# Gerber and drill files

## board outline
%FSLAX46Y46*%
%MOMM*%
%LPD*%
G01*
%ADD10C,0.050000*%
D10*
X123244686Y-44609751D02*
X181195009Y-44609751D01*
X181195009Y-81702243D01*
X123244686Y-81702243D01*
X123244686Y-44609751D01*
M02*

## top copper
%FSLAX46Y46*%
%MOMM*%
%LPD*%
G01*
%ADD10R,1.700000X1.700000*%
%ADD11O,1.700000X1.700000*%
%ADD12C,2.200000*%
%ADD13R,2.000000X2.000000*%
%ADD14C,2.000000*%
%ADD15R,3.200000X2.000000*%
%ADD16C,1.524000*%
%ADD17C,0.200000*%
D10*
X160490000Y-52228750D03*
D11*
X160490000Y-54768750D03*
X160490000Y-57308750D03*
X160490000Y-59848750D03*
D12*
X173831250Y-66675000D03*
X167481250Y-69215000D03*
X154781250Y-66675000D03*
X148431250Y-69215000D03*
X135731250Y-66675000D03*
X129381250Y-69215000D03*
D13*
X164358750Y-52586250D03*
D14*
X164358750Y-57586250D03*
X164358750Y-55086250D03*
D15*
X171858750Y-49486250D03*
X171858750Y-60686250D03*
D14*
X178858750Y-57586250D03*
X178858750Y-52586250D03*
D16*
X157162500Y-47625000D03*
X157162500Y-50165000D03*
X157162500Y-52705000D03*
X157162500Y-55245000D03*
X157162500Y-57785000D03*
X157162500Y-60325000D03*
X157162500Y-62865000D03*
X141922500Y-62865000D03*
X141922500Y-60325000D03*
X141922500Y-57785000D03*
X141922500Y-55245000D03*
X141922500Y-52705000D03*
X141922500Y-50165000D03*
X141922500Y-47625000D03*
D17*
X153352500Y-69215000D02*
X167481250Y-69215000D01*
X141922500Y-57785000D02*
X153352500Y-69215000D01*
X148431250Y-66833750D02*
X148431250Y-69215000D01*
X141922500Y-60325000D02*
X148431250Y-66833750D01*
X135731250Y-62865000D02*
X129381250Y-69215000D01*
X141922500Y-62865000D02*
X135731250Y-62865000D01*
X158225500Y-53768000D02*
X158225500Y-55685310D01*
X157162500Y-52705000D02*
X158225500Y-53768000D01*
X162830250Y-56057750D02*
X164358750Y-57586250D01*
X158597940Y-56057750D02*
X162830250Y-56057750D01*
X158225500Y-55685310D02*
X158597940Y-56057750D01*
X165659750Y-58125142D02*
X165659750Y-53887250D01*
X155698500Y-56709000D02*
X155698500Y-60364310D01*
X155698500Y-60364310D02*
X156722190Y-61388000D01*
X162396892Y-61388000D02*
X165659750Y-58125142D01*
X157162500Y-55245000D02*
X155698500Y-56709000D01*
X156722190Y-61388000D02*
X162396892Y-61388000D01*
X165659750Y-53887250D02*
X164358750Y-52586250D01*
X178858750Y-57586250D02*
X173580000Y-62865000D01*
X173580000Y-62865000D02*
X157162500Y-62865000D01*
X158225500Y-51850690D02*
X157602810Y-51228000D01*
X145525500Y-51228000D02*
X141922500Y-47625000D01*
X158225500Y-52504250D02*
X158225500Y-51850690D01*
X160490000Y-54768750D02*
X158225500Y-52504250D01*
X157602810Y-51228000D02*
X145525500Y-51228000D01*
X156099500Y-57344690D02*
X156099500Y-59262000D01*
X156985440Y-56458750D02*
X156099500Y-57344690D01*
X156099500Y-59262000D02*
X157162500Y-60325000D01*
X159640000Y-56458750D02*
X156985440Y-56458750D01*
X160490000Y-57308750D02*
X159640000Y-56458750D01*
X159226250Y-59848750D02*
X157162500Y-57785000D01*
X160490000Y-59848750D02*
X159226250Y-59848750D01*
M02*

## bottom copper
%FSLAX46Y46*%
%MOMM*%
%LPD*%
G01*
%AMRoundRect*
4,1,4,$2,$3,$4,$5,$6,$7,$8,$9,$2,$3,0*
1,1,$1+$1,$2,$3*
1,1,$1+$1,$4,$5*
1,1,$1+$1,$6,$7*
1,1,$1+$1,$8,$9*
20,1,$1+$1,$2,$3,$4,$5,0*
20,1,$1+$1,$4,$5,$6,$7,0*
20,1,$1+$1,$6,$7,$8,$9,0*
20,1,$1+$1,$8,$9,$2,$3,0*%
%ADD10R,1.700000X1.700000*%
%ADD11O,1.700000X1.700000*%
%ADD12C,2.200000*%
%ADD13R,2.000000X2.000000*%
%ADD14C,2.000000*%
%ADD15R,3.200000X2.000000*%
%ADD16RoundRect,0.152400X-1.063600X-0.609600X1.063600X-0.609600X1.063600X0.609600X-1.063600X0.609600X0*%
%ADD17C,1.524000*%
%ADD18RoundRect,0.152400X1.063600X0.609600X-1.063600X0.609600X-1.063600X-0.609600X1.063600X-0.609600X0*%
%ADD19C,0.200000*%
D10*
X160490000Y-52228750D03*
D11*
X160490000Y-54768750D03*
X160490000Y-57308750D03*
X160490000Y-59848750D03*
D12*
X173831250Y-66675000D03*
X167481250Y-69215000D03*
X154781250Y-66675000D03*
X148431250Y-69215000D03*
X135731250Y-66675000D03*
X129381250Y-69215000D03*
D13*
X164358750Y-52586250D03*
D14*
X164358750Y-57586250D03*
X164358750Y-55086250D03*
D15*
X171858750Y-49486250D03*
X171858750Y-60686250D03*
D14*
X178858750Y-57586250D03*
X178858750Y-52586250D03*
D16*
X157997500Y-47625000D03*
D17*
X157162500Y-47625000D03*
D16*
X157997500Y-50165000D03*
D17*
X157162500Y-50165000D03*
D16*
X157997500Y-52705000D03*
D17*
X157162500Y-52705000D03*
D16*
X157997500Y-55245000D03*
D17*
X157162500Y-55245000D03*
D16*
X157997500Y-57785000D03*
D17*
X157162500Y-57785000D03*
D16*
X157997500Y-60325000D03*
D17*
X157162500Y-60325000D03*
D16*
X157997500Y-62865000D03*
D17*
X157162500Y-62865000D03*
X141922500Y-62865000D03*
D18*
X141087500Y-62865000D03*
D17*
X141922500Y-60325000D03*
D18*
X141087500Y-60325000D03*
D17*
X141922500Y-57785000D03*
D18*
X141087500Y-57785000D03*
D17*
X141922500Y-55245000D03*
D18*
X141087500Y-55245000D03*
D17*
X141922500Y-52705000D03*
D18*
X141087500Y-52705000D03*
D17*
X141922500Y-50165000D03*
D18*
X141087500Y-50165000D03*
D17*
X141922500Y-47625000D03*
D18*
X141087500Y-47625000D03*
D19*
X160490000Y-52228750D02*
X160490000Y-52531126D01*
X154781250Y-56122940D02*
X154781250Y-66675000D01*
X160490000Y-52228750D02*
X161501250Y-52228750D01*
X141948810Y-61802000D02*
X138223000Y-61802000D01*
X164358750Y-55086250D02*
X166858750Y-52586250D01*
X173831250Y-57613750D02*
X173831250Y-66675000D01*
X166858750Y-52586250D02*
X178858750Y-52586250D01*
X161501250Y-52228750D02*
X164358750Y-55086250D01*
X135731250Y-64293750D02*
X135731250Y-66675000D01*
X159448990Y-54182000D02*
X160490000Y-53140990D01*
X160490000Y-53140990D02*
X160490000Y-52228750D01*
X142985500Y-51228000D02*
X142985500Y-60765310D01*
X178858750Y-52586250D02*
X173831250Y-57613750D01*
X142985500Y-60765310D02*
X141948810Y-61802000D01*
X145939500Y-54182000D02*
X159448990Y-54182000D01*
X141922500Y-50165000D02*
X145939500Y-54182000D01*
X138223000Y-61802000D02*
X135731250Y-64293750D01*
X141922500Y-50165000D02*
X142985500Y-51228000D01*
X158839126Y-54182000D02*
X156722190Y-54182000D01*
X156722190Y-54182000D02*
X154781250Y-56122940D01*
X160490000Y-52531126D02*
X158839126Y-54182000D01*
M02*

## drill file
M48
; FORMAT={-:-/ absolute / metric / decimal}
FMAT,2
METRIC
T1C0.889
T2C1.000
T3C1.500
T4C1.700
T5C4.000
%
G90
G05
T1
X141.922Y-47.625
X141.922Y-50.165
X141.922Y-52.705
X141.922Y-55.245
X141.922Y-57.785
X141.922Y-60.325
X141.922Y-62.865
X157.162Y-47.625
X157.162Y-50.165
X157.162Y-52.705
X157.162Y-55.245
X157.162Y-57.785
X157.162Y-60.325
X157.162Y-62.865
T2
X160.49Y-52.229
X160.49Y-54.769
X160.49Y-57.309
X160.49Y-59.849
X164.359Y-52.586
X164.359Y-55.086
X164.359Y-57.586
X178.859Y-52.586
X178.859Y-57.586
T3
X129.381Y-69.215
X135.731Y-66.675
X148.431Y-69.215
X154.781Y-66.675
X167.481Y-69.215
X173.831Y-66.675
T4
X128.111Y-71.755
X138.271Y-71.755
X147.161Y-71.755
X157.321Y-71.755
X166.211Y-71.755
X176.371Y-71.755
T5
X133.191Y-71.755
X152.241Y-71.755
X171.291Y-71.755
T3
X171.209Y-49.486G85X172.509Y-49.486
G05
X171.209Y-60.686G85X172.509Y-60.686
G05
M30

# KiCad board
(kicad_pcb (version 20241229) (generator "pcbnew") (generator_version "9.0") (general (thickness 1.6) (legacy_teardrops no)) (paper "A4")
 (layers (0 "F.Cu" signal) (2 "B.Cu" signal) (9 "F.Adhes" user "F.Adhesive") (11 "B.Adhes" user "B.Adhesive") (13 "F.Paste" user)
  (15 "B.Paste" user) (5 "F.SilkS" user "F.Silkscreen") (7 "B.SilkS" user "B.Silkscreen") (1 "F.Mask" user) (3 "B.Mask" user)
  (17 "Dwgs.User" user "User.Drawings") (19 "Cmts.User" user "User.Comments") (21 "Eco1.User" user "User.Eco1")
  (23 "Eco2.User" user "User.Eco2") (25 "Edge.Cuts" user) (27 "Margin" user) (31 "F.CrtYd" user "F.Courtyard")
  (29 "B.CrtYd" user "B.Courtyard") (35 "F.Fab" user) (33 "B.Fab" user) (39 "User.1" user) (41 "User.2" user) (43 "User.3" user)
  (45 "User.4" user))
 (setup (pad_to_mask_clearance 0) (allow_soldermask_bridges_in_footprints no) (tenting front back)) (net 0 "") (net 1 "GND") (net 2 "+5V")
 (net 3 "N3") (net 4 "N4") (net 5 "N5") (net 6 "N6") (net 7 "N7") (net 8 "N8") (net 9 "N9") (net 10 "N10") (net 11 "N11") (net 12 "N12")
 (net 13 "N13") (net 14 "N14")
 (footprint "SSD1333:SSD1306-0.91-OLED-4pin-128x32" (layer "F.Cu") (at 123.99 50.03875)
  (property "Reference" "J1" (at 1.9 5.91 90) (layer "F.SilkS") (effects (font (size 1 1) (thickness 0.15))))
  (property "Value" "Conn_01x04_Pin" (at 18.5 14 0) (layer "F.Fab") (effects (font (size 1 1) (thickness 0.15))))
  (pad "1" thru_hole rect (at 36.5 2.19) (size 1.7 1.7) (drill 1) (layers "*.Cu" "*.Mask") (remove_unused_layers no) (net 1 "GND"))
  (pad "2" thru_hole oval (at 36.5 4.73) (size 1.7 1.7) (drill 1) (layers "*.Cu" "*.Mask") (remove_unused_layers no) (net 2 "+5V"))
  (pad "3" thru_hole oval (at 36.5 7.27) (size 1.7 1.7) (drill 1) (layers "*.Cu" "*.Mask") (remove_unused_layers no) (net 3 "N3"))
  (pad "4" thru_hole oval (at 36.5 9.81) (size 1.7 1.7) (drill 1) (layers "*.Cu" "*.Mask") (remove_unused_layers no) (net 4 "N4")))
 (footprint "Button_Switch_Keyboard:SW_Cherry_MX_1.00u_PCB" (layer "F.Cu") (at 173.83125 66.675)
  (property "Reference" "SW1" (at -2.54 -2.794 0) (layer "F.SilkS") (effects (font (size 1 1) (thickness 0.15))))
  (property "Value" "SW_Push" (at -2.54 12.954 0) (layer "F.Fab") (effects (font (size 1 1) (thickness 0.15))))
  (pad "" np_thru_hole circle (at -7.62 5.08) (size 1.7 1.7) (drill 1.7) (layers "*.Cu" "*.Mask"))
  (pad "" np_thru_hole circle (at -2.54 5.08) (size 4 4) (drill 4) (layers "*.Cu" "*.Mask"))
  (pad "" np_thru_hole circle (at 2.54 5.08) (size 1.7 1.7) (drill 1.7) (layers "*.Cu" "*.Mask"))
  (pad "1" thru_hole circle (at 0 0) (size 2.2 2.2) (drill 1.5) (layers "*.Cu" "*.Mask") (remove_unused_layers no) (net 1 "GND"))
  (pad "2" thru_hole circle (at -6.35 2.54) (size 2.2 2.2) (drill 1.5) (layers "*.Cu" "*.Mask") (remove_unused_layers no) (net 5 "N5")))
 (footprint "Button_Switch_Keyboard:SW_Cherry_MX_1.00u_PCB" (layer "F.Cu") (at 154.78125 66.675)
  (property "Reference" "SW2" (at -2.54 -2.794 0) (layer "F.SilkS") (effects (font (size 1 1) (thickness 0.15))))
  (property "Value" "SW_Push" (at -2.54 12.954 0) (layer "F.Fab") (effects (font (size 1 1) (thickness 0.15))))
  (pad "" np_thru_hole circle (at -7.62 5.08) (size 1.7 1.7) (drill 1.7) (layers "*.Cu" "*.Mask"))
  (pad "" np_thru_hole circle (at -2.54 5.08) (size 4 4) (drill 4) (layers "*.Cu" "*.Mask"))
  (pad "" np_thru_hole circle (at 2.54 5.08) (size 1.7 1.7) (drill 1.7) (layers "*.Cu" "*.Mask"))
  (pad "1" thru_hole circle (at 0 0) (size 2.2 2.2) (drill 1.5) (layers "*.Cu" "*.Mask") (remove_unused_layers no) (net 1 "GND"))
  (pad "2" thru_hole circle (at -6.35 2.54) (size 2.2 2.2) (drill 1.5) (layers "*.Cu" "*.Mask") (remove_unused_layers no) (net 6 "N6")))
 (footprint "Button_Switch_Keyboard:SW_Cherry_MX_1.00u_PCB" (layer "F.Cu") (at 135.73125 66.675)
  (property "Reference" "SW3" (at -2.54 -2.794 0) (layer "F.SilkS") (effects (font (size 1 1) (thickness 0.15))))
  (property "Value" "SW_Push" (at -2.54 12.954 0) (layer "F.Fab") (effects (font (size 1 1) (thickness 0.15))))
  (pad "" np_thru_hole circle (at -7.62 5.08) (size 1.7 1.7) (drill 1.7) (layers "*.Cu" "*.Mask"))
  (pad "" np_thru_hole circle (at -2.54 5.08) (size 4 4) (drill 4) (layers "*.Cu" "*.Mask"))
  (pad "" np_thru_hole circle (at 2.54 5.08) (size 1.7 1.7) (drill 1.7) (layers "*.Cu" "*.Mask"))
  (pad "1" thru_hole circle (at 0 0) (size 2.2 2.2) (drill 1.5) (layers "*.Cu" "*.Mask") (remove_unused_layers no) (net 1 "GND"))
  (pad "2" thru_hole circle (at -6.35 2.54) (size 2.2 2.2) (drill 1.5) (layers "*.Cu" "*.Mask") (remove_unused_layers no) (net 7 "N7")))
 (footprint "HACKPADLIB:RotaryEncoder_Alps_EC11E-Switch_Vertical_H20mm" (layer "F.Cu") (at 164.35875 52.58625)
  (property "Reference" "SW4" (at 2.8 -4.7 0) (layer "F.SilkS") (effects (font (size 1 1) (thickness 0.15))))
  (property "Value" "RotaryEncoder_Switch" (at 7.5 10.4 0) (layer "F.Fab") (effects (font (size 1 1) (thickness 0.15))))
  (pad "A" thru_hole rect (at 0 0) (size 2 2) (drill 1) (layers "*.Cu" "*.Mask") (remove_unused_layers no) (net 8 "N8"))
  (pad "B" thru_hole circle (at 0 5) (size 2 2) (drill 1) (layers "*.Cu" "*.Mask") (remove_unused_layers no) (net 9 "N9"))
  (pad "C" thru_hole circle (at 0 2.5) (size 2 2) (drill 1) (layers "*.Cu" "*.Mask") (remove_unused_layers no) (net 1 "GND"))
  (pad "MP" thru_hole rect (at 7.5 -3.1) (size 3.2 2) (drill oval 2.8 1.5) (layers "*.Cu" "*.Mask") (remove_unused_layers no))
  (pad "MP" thru_hole rect (at 7.5 8.1) (size 3.2 2) (drill oval 2.8 1.5) (layers "*.Cu" "*.Mask") (remove_unused_layers no))
  (pad "S1" thru_hole circle (at 14.5 5) (size 2 2) (drill 1) (layers "*.Cu" "*.Mask") (remove_unused_layers no) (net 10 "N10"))
  (pad "S2" thru_hole circle (at 14.5 0) (size 2 2) (drill 1) (layers "*.Cu" "*.Mask") (remove_unused_layers no) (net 1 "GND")))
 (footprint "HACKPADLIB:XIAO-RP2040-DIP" (layer "B.Cu") (at 149.5425 55.245 180)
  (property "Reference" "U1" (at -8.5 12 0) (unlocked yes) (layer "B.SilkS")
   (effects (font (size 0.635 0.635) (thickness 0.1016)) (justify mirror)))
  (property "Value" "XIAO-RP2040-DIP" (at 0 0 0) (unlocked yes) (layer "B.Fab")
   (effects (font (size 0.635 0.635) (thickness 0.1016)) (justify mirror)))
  (pad "1" smd roundrect (at -8.455 7.62) (size 2.432 1.524) (layers "B.Cu" "B.Mask") (roundrect_rratio 0.1) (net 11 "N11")
   (thermal_bridge_angle 45))
  (pad "1" thru_hole circle (at -7.62 7.62) (size 1.524 1.524) (drill 0.889) (layers "*.Cu" "*.Mask") (remove_unused_layers no)
   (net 11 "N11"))
  (pad "2" smd roundrect (at -8.455 5.08) (size 2.432 1.524) (layers "B.Cu" "B.Mask") (roundrect_rratio 0.1) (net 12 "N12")
   (thermal_bridge_angle 45))
  (pad "2" thru_hole circle (at -7.62 5.08) (size 1.524 1.524) (drill 0.889) (layers "*.Cu" "*.Mask") (remove_unused_layers no)
   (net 12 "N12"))
  (pad "3" smd roundrect (at -8.455 2.54) (size 2.432 1.524) (layers "B.Cu" "B.Mask") (roundrect_rratio 0.1) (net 9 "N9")
   (thermal_bridge_angle 45))
  (pad "3" thru_hole circle (at -7.62 2.54) (size 1.524 1.524) (drill 0.889) (layers "*.Cu" "*.Mask") (remove_unused_layers no) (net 9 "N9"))
  (pad "4" smd roundrect (at -8.455 0) (size 2.432 1.524) (layers "B.Cu" "B.Mask") (roundrect_rratio 0.1) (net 8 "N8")
   (thermal_bridge_angle 45))
  (pad "4" thru_hole circle (at -7.62 0) (size 1.524 1.524) (drill 0.889) (layers "*.Cu" "*.Mask") (remove_unused_layers no) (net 8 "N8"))
  (pad "5" smd roundrect (at -8.455 -2.54) (size 2.432 1.524) (layers "B.Cu" "B.Mask") (roundrect_rratio 0.1) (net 4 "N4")
   (thermal_bridge_angle 45))
  (pad "5" thru_hole circle (at -7.62 -2.54) (size 1.524 1.524) (drill 0.889) (layers "*.Cu" "*.Mask") (remove_unused_layers no)
   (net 4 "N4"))
  (pad "6" smd roundrect (at -8.455 -5.08) (size 2.432 1.524) (layers "B.Cu" "B.Mask") (roundrect_rratio 0.1) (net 3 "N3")
   (thermal_bridge_angle 45))
  (pad "6" thru_hole circle (at -7.62 -5.08) (size 1.524 1.524) (drill 0.889) (layers "*.Cu" "*.Mask") (remove_unused_layers no)
   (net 3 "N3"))
  (pad "7" smd roundrect (at -8.455 -7.62) (size 2.432 1.524) (layers "B.Cu" "B.Mask") (roundrect_rratio 0.1) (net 10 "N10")
   (thermal_bridge_angle 45))
  (pad "7" thru_hole circle (at -7.62 -7.62) (size 1.524 1.524) (drill 0.889) (layers "*.Cu" "*.Mask") (remove_unused_layers no)
   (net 10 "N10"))
  (pad "8" thru_hole circle (at 7.62 -7.62 180) (size 1.524 1.524) (drill 0.889) (layers "*.Cu" "*.Mask") (remove_unused_layers no)
   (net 7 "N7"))
  (pad "8" smd roundrect (at 8.455 -7.62 180) (size 2.432 1.524) (layers "B.Cu" "B.Mask") (roundrect_rratio 0.1) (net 7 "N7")
   (thermal_bridge_angle 45))
  (pad "9" thru_hole circle (at 7.62 -5.08 180) (size 1.524 1.524) (drill 0.889) (layers "*.Cu" "*.Mask") (remove_unused_layers no)
   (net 6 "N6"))
  (pad "9" smd roundrect (at 8.455 -5.08 180) (size 2.432 1.524) (layers "B.Cu" "B.Mask") (roundrect_rratio 0.1) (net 6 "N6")
   (thermal_bridge_angle 45))
  (pad "10" thru_hole circle (at 7.62 -2.54 180) (size 1.524 1.524) (drill 0.889) (layers "*.Cu" "*.Mask") (remove_unused_layers no)
   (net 5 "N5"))
  (pad "10" smd roundrect (at 8.455 -2.54 180) (size 2.432 1.524) (layers "B.Cu" "B.Mask") (roundrect_rratio 0.1) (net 5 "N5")
   (thermal_bridge_angle 45))
  (pad "11" thru_hole circle (at 7.62 0 180) (size 1.524 1.524) (drill 0.889) (layers "*.Cu" "*.Mask") (remove_unused_layers no)
   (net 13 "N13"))
  (pad "11" smd roundrect (at 8.455 0 180) (size 2.432 1.524) (layers "B.Cu" "B.Mask") (roundrect_rratio 0.1) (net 13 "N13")
   (thermal_bridge_angle 45))
  (pad "12" thru_hole circle (at 7.62 2.54 180) (size 1.524 1.524) (drill 0.889) (layers "*.Cu" "*.Mask") (remove_unused_layers no)
   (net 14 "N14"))
  (pad "12" smd roundrect (at 8.455 2.54 180) (size 2.432 1.524) (layers "B.Cu" "B.Mask") (roundrect_rratio 0.1) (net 14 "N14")
   (thermal_bridge_angle 45))
  (pad "13" thru_hole circle (at 7.62 5.08 180) (size 1.524 1.524) (drill 0.889) (layers "*.Cu" "*.Mask") (remove_unused_layers no)
   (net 1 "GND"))
  (pad "13" smd roundrect (at 8.455 5.08 180) (size 2.432 1.524) (layers "B.Cu" "B.Mask") (roundrect_rratio 0.1) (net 1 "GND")
   (thermal_bridge_angle 45))
  (pad "14" thru_hole circle (at 7.62 7.62 180) (size 1.524 1.524) (drill 0.889) (layers "*.Cu" "*.Mask") (remove_unused_layers no)
   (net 2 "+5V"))
  (pad "14" smd roundrect (at 8.455 7.62 180) (size 2.432 1.524) (layers "B.Cu" "B.Mask") (roundrect_rratio 0.1) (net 2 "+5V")
   (thermal_bridge_angle 45)))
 (gr_rect (start 123.244686 44.609751) (end 181.195009 81.702243) (stroke (width 0.05) (type default)) (fill no) (layer "Edge.Cuts"))
 (segment (start 153.3525 69.215) (end 167.48125 69.215) (width 0.2) (layer "F.Cu") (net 5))
 (segment (start 141.9225 57.785) (end 153.3525 69.215) (width 0.2) (layer "F.Cu") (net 5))
 (segment (start 160.49 52.22875) (end 160.49 52.531126) (width 0.2) (layer "B.Cu") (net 1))
 (segment (start 154.78125 56.12294) (end 154.78125 66.675) (width 0.2) (layer "B.Cu") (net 1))
 (segment (start 160.49 52.22875) (end 161.50125 52.22875) (width 0.2) (layer "B.Cu") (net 1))
 (segment (start 141.94881 61.802) (end 138.223 61.802) (width 0.2) (layer "B.Cu") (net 1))
 (segment (start 164.35875 55.08625) (end 166.85875 52.58625) (width 0.2) (layer "B.Cu") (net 1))
 (segment (start 173.83125 57.61375) (end 173.83125 66.675) (width 0.2) (layer "B.Cu") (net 1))
 (segment (start 166.85875 52.58625) (end 178.85875 52.58625) (width 0.2) (layer "B.Cu") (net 1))
 (segment (start 161.50125 52.22875) (end 164.35875 55.08625) (width 0.2) (layer "B.Cu") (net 1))
 (segment (start 135.73125 64.29375) (end 135.73125 66.675) (width 0.2) (layer "B.Cu") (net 1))
 (segment (start 159.44899 54.182) (end 160.49 53.14099) (width 0.2) (layer "B.Cu") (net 1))
 (segment (start 160.49 53.14099) (end 160.49 52.22875) (width 0.2) (layer "B.Cu") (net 1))
 (segment (start 142.9855 51.228) (end 142.9855 60.76531) (width 0.2) (layer "B.Cu") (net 1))
 (segment (start 178.85875 52.58625) (end 173.83125 57.61375) (width 0.2) (layer "B.Cu") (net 1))
 (segment (start 142.9855 60.76531) (end 141.94881 61.802) (width 0.2) (layer "B.Cu") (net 1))
 (segment (start 145.9395 54.182) (end 159.44899 54.182) (width 0.2) (layer "B.Cu") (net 1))
 (segment (start 141.9225 50.165) (end 145.9395 54.182) (width 0.2) (layer "B.Cu") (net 1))
 (segment (start 138.223 61.802) (end 135.73125 64.29375) (width 0.2) (layer "B.Cu") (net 1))
 (segment (start 141.9225 50.165) (end 142.9855 51.228) (width 0.2) (layer "B.Cu") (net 1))
 (segment (start 158.839126 54.182) (end 156.72219 54.182) (width 0.2) (layer "B.Cu") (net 1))
 (segment (start 156.72219 54.182) (end 154.78125 56.12294) (width 0.2) (layer "B.Cu") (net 1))
 (segment (start 160.49 52.531126) (end 158.839126 54.182) (width 0.2) (layer "B.Cu") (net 1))
 (segment (start 148.43125 66.83375) (end 148.43125 69.215) (width 0.2) (layer "F.Cu") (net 6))
 (segment (start 141.9225 60.325) (end 148.43125 66.83375) (width 0.2) (layer "F.Cu") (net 6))
 (segment (start 135.73125 62.865) (end 129.38125 69.215) (width 0.2) (layer "F.Cu") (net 7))
 (segment (start 141.9225 62.865) (end 135.73125 62.865) (width 0.2) (layer "F.Cu") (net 7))
 (segment (start 158.2255 53.768) (end 158.2255 55.68531) (width 0.2) (layer "F.Cu") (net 9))
 (segment (start 157.1625 52.705) (end 158.2255 53.768) (width 0.2) (layer "F.Cu") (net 9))
 (segment (start 162.83025 56.05775) (end 164.35875 57.58625) (width 0.2) (layer "F.Cu") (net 9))
 (segment (start 158.59794 56.05775) (end 162.83025 56.05775) (width 0.2) (layer "F.Cu") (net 9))
 (segment (start 158.2255 55.68531) (end 158.59794 56.05775) (width 0.2) (layer "F.Cu") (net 9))
 (segment (start 165.65975 58.125142) (end 165.65975 53.88725) (width 0.2) (layer "F.Cu") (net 8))
 (segment (start 155.6985 56.709) (end 155.6985 60.36431) (width 0.2) (layer "F.Cu") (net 8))
 (segment (start 155.6985 60.36431) (end 156.72219 61.388) (width 0.2) (layer "F.Cu") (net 8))
 (segment (start 162.396892 61.388) (end 165.65975 58.125142) (width 0.2) (layer "F.Cu") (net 8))
 (segment (start 157.1625 55.245) (end 155.6985 56.709) (width 0.2) (layer "F.Cu") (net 8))
 (segment (start 156.72219 61.388) (end 162.396892 61.388) (width 0.2) (layer "F.Cu") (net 8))
 (segment (start 165.65975 53.88725) (end 164.35875 52.58625) (width 0.2) (layer "F.Cu") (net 8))
 (segment (start 178.85875 57.58625) (end 173.58 62.865) (width 0.2) (layer "F.Cu") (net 10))
 (segment (start 173.58 62.865) (end 157.1625 62.865) (width 0.2) (layer "F.Cu") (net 10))
 (segment (start 158.2255 51.85069) (end 157.60281 51.228) (width 0.2) (layer "F.Cu") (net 2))
 (segment (start 145.5255 51.228) (end 141.9225 47.625) (width 0.2) (layer "F.Cu") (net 2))
 (segment (start 158.2255 52.50425) (end 158.2255 51.85069) (width 0.2) (layer "F.Cu") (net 2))
 (segment (start 160.49 54.76875) (end 158.2255 52.50425) (width 0.2) (layer "F.Cu") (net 2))
 (segment (start 157.60281 51.228) (end 145.5255 51.228) (width 0.2) (layer "F.Cu") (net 2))
 (segment (start 156.0995 57.34469) (end 156.0995 59.262) (width 0.2) (layer "F.Cu") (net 3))
 (segment (start 156.98544 56.45875) (end 156.0995 57.34469) (width 0.2) (layer "F.Cu") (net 3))
 (segment (start 156.0995 59.262) (end 157.1625 60.325) (width 0.2) (layer "F.Cu") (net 3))
 (segment (start 159.64 56.45875) (end 156.98544 56.45875) (width 0.2) (layer "F.Cu") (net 3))
 (segment (start 160.49 57.30875) (end 159.64 56.45875) (width 0.2) (layer "F.Cu") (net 3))
 (segment (start 159.22625 59.84875) (end 157.1625 57.785) (width 0.2) (layer "F.Cu") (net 4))
 (segment (start 160.49 59.84875) (end 159.22625 59.84875) (width 0.2) (layer "F.Cu") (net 4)))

